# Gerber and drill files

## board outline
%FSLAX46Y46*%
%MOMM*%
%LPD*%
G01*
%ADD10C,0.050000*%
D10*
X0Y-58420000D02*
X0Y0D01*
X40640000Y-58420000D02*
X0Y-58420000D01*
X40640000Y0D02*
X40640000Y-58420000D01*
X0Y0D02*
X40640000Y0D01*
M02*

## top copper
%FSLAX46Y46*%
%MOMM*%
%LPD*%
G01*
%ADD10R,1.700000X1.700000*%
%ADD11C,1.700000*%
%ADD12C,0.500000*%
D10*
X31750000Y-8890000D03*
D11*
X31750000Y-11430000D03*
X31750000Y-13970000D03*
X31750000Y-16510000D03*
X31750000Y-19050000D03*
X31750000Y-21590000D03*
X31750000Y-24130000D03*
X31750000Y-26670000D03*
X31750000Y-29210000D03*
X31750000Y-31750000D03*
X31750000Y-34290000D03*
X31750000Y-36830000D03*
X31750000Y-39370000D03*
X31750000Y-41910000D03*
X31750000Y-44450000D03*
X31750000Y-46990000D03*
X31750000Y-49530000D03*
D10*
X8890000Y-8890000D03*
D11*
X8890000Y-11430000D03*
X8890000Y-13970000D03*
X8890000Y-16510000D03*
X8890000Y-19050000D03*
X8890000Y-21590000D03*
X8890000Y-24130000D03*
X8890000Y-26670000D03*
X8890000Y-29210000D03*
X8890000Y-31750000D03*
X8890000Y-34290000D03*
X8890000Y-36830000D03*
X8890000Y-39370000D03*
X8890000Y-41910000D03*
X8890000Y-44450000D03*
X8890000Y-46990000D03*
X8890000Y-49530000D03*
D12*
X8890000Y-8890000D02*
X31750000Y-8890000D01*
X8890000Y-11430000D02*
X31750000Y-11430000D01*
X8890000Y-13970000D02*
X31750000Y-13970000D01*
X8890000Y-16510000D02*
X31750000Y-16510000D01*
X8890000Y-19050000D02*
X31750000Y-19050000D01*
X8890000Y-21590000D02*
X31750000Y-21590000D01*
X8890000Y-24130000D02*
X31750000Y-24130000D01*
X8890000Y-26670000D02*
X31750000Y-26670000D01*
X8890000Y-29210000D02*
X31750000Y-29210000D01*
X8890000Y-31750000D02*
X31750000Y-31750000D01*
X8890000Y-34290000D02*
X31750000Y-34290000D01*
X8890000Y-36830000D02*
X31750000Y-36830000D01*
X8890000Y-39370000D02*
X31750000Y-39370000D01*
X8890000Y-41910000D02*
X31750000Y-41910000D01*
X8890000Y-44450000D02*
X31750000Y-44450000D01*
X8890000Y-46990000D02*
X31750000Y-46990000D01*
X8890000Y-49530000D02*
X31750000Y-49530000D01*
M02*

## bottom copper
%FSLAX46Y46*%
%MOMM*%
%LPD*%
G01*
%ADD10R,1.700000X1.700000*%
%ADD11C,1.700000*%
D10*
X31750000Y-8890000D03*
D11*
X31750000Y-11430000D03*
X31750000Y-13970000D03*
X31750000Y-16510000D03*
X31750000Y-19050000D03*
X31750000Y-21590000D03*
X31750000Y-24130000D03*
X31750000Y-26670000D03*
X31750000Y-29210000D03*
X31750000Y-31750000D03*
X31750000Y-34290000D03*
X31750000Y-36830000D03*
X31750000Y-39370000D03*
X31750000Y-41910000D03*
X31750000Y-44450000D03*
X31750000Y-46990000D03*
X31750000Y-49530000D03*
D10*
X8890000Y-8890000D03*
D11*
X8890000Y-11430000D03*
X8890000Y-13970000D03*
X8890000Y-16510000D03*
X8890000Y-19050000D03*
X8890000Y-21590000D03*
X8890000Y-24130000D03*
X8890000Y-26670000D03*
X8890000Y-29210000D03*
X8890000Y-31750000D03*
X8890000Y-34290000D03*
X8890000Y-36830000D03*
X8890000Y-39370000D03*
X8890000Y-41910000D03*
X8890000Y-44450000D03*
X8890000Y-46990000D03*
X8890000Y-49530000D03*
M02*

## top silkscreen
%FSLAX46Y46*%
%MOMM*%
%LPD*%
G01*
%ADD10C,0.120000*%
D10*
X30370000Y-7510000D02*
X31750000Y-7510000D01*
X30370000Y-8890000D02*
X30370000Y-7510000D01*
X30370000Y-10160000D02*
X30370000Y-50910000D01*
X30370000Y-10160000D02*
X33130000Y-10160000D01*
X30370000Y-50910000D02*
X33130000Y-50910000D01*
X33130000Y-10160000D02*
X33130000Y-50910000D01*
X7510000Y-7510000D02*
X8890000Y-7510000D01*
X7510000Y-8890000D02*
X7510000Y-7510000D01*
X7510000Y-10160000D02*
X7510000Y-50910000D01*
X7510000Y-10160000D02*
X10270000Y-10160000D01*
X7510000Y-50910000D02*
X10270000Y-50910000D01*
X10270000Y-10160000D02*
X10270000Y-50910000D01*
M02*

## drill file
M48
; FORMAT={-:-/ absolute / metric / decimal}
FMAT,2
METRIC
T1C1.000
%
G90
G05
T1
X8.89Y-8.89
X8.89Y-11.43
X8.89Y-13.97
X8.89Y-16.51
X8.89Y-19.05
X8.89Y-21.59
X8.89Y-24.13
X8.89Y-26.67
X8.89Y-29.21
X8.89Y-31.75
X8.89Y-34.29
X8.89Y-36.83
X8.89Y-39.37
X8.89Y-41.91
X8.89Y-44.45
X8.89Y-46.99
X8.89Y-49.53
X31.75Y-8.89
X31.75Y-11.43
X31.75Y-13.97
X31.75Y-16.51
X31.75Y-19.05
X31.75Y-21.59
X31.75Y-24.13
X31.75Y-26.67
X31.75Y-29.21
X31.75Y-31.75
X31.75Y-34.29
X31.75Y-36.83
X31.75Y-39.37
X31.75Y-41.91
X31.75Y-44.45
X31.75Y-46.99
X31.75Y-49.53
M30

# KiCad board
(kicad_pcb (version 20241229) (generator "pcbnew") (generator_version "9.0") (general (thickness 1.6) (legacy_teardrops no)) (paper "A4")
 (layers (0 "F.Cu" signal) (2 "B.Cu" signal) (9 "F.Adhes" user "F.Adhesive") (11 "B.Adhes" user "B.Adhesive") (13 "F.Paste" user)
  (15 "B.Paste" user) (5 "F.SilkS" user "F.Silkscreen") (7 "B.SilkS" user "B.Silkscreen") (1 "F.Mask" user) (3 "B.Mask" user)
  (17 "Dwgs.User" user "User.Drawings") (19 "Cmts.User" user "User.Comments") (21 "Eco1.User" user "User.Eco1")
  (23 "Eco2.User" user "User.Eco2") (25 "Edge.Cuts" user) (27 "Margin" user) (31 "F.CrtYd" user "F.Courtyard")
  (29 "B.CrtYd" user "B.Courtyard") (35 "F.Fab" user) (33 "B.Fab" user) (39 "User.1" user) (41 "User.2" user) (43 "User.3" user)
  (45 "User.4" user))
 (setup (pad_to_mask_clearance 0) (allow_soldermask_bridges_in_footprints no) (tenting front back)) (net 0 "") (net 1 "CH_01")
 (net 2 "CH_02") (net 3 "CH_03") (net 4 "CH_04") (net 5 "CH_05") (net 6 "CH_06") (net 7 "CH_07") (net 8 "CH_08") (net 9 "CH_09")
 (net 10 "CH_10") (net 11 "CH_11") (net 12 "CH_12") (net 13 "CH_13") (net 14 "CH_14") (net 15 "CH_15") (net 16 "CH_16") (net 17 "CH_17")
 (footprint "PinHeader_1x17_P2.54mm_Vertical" (layer "F.Cu") (at 31.75 8.89)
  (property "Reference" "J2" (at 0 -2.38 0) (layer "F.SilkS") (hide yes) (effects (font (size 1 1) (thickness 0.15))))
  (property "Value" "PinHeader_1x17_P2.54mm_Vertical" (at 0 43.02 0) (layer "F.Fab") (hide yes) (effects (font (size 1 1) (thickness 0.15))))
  (fp_line (start -1.38 -1.38) (end 0 -1.38) (stroke (width 0.12) (type solid)) (layer "F.SilkS"))
  (fp_line (start -1.38 0) (end -1.38 -1.38) (stroke (width 0.12) (type solid)) (layer "F.SilkS"))
  (fp_line (start -1.38 1.27) (end -1.38 42.02) (stroke (width 0.12) (type solid)) (layer "F.SilkS"))
  (fp_line (start -1.38 1.27) (end 1.38 1.27) (stroke (width 0.12) (type solid)) (layer "F.SilkS"))
  (fp_line (start -1.38 42.02) (end 1.38 42.02) (stroke (width 0.12) (type solid)) (layer "F.SilkS"))
  (fp_line (start 1.38 1.27) (end 1.38 42.02) (stroke (width 0.12) (type solid)) (layer "F.SilkS"))
  (pad "1" thru_hole rect (at 0 0) (size 1.7 1.7) (drill 1) (layers "*.Cu" "*.Mask") (remove_unused_layers no) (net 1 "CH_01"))
  (pad "2" thru_hole circle (at 0 2.54) (size 1.7 1.7) (drill 1) (layers "*.Cu" "*.Mask") (remove_unused_layers no) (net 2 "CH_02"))
  (pad "3" thru_hole circle (at 0 5.08) (size 1.7 1.7) (drill 1) (layers "*.Cu" "*.Mask") (remove_unused_layers no) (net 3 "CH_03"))
  (pad "4" thru_hole circle (at 0 7.62) (size 1.7 1.7) (drill 1) (layers "*.Cu" "*.Mask") (remove_unused_layers no) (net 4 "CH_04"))
  (pad "5" thru_hole circle (at 0 10.16) (size 1.7 1.7) (drill 1) (layers "*.Cu" "*.Mask") (remove_unused_layers no) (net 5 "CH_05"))
  (pad "6" thru_hole circle (at 0 12.7) (size 1.7 1.7) (drill 1) (layers "*.Cu" "*.Mask") (remove_unused_layers no) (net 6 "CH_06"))
  (pad "7" thru_hole circle (at 0 15.24) (size 1.7 1.7) (drill 1) (layers "*.Cu" "*.Mask") (remove_unused_layers no) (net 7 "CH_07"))
  (pad "8" thru_hole circle (at 0 17.78) (size 1.7 1.7) (drill 1) (layers "*.Cu" "*.Mask") (remove_unused_layers no) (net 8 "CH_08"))
  (pad "9" thru_hole circle (at 0 20.32) (size 1.7 1.7) (drill 1) (layers "*.Cu" "*.Mask") (remove_unused_layers no) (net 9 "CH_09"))
  (pad "10" thru_hole circle (at 0 22.86) (size 1.7 1.7) (drill 1) (layers "*.Cu" "*.Mask") (remove_unused_layers no) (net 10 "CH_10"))
  (pad "11" thru_hole circle (at 0 25.4) (size 1.7 1.7) (drill 1) (layers "*.Cu" "*.Mask") (remove_unused_layers no) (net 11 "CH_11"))
  (pad "12" thru_hole circle (at 0 27.94) (size 1.7 1.7) (drill 1) (layers "*.Cu" "*.Mask") (remove_unused_layers no) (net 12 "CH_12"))
  (pad "13" thru_hole circle (at 0 30.48) (size 1.7 1.7) (drill 1) (layers "*.Cu" "*.Mask") (remove_unused_layers no) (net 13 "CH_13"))
  (pad "14" thru_hole circle (at 0 33.02) (size 1.7 1.7) (drill 1) (layers "*.Cu" "*.Mask") (remove_unused_layers no) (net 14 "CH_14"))
  (pad "15" thru_hole circle (at 0 35.56) (size 1.7 1.7) (drill 1) (layers "*.Cu" "*.Mask") (remove_unused_layers no) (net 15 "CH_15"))
  (pad "16" thru_hole circle (at 0 38.1) (size 1.7 1.7) (drill 1) (layers "*.Cu" "*.Mask") (remove_unused_layers no) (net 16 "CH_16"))
  (pad "17" thru_hole circle (at 0 40.64) (size 1.7 1.7) (drill 1) (layers "*.Cu" "*.Mask") (remove_unused_layers no) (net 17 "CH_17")))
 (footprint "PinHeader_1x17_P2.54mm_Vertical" (layer "F.Cu") (at 8.89 8.89)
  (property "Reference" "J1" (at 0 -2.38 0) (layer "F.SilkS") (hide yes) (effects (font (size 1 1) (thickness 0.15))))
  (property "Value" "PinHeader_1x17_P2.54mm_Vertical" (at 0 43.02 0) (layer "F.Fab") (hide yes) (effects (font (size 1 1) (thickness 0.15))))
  (fp_line (start -1.38 -1.38) (end 0 -1.38) (stroke (width 0.12) (type solid)) (layer "F.SilkS"))
  (fp_line (start -1.38 0) (end -1.38 -1.38) (stroke (width 0.12) (type solid)) (layer "F.SilkS"))
  (fp_line (start -1.38 1.27) (end -1.38 42.02) (stroke (width 0.12) (type solid)) (layer "F.SilkS"))
  (fp_line (start -1.38 1.27) (end 1.38 1.27) (stroke (width 0.12) (type solid)) (layer "F.SilkS"))
  (fp_line (start -1.38 42.02) (end 1.38 42.02) (stroke (width 0.12) (type solid)) (layer "F.SilkS"))
  (fp_line (start 1.38 1.27) (end 1.38 42.02) (stroke (width 0.12) (type solid)) (layer "F.SilkS"))
  (pad "1" thru_hole rect (at 0 0) (size 1.7 1.7) (drill 1) (layers "*.Cu" "*.Mask") (remove_unused_layers no) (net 1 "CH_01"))
  (pad "2" thru_hole circle (at 0 2.54) (size 1.7 1.7) (drill 1) (layers "*.Cu" "*.Mask") (remove_unused_layers no) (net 2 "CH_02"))
  (pad "3" thru_hole circle (at 0 5.08) (size 1.7 1.7) (drill 1) (layers "*.Cu" "*.Mask") (remove_unused_layers no) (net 3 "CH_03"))
  (pad "4" thru_hole circle (at 0 7.62) (size 1.7 1.7) (drill 1) (layers "*.Cu" "*.Mask") (remove_unused_layers no) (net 4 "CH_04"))
  (pad "5" thru_hole circle (at 0 10.16) (size 1.7 1.7) (drill 1) (layers "*.Cu" "*.Mask") (remove_unused_layers no) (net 5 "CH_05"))
  (pad "6" thru_hole circle (at 0 12.7) (size 1.7 1.7) (drill 1) (layers "*.Cu" "*.Mask") (remove_unused_layers no) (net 6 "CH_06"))
  (pad "7" thru_hole circle (at 0 15.24) (size 1.7 1.7) (drill 1) (layers "*.Cu" "*.Mask") (remove_unused_layers no) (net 7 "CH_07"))
  (pad "8" thru_hole circle (at 0 17.78) (size 1.7 1.7) (drill 1) (layers "*.Cu" "*.Mask") (remove_unused_layers no) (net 8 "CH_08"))
  (pad "9" thru_hole circle (at 0 20.32) (size 1.7 1.7) (drill 1) (layers "*.Cu" "*.Mask") (remove_unused_layers no) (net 9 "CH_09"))
  (pad "10" thru_hole circle (at 0 22.86) (size 1.7 1.7) (drill 1) (layers "*.Cu" "*.Mask") (remove_unused_layers no) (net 10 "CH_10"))
  (pad "11" thru_hole circle (at 0 25.4) (size 1.7 1.7) (drill 1) (layers "*.Cu" "*.Mask") (remove_unused_layers no) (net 11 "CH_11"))
  (pad "12" thru_hole circle (at 0 27.94) (size 1.7 1.7) (drill 1) (layers "*.Cu" "*.Mask") (remove_unused_layers no) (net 12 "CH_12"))
  (pad "13" thru_hole circle (at 0 30.48) (size 1.7 1.7) (drill 1) (layers "*.Cu" "*.Mask") (remove_unused_layers no) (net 13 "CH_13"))
  (pad "14" thru_hole circle (at 0 33.02) (size 1.7 1.7) (drill 1) (layers "*.Cu" "*.Mask") (remove_unused_layers no) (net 14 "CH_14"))
  (pad "15" thru_hole circle (at 0 35.56) (size 1.7 1.7) (drill 1) (layers "*.Cu" "*.Mask") (remove_unused_layers no) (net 15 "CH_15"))
  (pad "16" thru_hole circle (at 0 38.1) (size 1.7 1.7) (drill 1) (layers "*.Cu" "*.Mask") (remove_unused_layers no) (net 16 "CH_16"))
  (pad "17" thru_hole circle (at 0 40.64) (size 1.7 1.7) (drill 1) (layers "*.Cu" "*.Mask") (remove_unused_layers no) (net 17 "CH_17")))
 (gr_line (start 0 58.42) (end 0 0) (stroke (width 0.05) (type default)) (layer "Edge.Cuts"))
 (gr_line (start 40.64 58.42) (end 0 58.42) (stroke (width 0.05) (type default)) (layer "Edge.Cuts"))
 (gr_line (start 40.64 0) (end 40.64 58.42) (stroke (width 0.05) (type default)) (layer "Edge.Cuts"))
 (gr_line (start 0 0) (end 40.64 0) (stroke (width 0.05) (type default)) (layer "Edge.Cuts"))
 (segment (start 8.89 8.89) (end 31.75 8.89) (width 0.5) (layer "F.Cu") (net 1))
 (segment (start 8.89 11.43) (end 31.75 11.43) (width 0.5) (layer "F.Cu") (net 2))
 (segment (start 8.89 13.97) (end 31.75 13.97) (width 0.5) (layer "F.Cu") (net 3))
 (segment (start 8.89 16.51) (end 31.75 16.51) (width 0.5) (layer "F.Cu") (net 4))
 (segment (start 8.89 19.05) (end 31.75 19.05) (width 0.5) (layer "F.Cu") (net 5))
 (segment (start 8.89 21.59) (end 31.75 21.59) (width 0.5) (layer "F.Cu") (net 6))
 (segment (start 8.89 24.13) (end 31.75 24.13) (width 0.5) (layer "F.Cu") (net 7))
 (segment (start 8.89 26.67) (end 31.75 26.67) (width 0.5) (layer "F.Cu") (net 8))
 (segment (start 8.89 29.21) (end 31.75 29.21) (width 0.5) (layer "F.Cu") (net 9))
 (segment (start 8.89 31.75) (end 31.75 31.75) (width 0.5) (layer "F.Cu") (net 10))
 (segment (start 8.89 34.29) (end 31.75 34.29) (width 0.5) (layer "F.Cu") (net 11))
 (segment (start 8.89 36.83) (end 31.75 36.83) (width 0.5) (layer "F.Cu") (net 12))
 (segment (start 8.89 39.37) (end 31.75 39.37) (width 0.5) (layer "F.Cu") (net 13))
 (segment (start 8.89 41.91) (end 31.75 41.91) (width 0.5) (layer "F.Cu") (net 14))
 (segment (start 8.89 44.45) (end 31.75 44.45) (width 0.5) (layer "F.Cu") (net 15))
 (segment (start 8.89 46.99) (end 31.75 46.99) (width 0.5) (layer "F.Cu") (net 16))
 (segment (start 8.89 49.53) (end 31.75 49.53) (width 0.5) (layer "F.Cu") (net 17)))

